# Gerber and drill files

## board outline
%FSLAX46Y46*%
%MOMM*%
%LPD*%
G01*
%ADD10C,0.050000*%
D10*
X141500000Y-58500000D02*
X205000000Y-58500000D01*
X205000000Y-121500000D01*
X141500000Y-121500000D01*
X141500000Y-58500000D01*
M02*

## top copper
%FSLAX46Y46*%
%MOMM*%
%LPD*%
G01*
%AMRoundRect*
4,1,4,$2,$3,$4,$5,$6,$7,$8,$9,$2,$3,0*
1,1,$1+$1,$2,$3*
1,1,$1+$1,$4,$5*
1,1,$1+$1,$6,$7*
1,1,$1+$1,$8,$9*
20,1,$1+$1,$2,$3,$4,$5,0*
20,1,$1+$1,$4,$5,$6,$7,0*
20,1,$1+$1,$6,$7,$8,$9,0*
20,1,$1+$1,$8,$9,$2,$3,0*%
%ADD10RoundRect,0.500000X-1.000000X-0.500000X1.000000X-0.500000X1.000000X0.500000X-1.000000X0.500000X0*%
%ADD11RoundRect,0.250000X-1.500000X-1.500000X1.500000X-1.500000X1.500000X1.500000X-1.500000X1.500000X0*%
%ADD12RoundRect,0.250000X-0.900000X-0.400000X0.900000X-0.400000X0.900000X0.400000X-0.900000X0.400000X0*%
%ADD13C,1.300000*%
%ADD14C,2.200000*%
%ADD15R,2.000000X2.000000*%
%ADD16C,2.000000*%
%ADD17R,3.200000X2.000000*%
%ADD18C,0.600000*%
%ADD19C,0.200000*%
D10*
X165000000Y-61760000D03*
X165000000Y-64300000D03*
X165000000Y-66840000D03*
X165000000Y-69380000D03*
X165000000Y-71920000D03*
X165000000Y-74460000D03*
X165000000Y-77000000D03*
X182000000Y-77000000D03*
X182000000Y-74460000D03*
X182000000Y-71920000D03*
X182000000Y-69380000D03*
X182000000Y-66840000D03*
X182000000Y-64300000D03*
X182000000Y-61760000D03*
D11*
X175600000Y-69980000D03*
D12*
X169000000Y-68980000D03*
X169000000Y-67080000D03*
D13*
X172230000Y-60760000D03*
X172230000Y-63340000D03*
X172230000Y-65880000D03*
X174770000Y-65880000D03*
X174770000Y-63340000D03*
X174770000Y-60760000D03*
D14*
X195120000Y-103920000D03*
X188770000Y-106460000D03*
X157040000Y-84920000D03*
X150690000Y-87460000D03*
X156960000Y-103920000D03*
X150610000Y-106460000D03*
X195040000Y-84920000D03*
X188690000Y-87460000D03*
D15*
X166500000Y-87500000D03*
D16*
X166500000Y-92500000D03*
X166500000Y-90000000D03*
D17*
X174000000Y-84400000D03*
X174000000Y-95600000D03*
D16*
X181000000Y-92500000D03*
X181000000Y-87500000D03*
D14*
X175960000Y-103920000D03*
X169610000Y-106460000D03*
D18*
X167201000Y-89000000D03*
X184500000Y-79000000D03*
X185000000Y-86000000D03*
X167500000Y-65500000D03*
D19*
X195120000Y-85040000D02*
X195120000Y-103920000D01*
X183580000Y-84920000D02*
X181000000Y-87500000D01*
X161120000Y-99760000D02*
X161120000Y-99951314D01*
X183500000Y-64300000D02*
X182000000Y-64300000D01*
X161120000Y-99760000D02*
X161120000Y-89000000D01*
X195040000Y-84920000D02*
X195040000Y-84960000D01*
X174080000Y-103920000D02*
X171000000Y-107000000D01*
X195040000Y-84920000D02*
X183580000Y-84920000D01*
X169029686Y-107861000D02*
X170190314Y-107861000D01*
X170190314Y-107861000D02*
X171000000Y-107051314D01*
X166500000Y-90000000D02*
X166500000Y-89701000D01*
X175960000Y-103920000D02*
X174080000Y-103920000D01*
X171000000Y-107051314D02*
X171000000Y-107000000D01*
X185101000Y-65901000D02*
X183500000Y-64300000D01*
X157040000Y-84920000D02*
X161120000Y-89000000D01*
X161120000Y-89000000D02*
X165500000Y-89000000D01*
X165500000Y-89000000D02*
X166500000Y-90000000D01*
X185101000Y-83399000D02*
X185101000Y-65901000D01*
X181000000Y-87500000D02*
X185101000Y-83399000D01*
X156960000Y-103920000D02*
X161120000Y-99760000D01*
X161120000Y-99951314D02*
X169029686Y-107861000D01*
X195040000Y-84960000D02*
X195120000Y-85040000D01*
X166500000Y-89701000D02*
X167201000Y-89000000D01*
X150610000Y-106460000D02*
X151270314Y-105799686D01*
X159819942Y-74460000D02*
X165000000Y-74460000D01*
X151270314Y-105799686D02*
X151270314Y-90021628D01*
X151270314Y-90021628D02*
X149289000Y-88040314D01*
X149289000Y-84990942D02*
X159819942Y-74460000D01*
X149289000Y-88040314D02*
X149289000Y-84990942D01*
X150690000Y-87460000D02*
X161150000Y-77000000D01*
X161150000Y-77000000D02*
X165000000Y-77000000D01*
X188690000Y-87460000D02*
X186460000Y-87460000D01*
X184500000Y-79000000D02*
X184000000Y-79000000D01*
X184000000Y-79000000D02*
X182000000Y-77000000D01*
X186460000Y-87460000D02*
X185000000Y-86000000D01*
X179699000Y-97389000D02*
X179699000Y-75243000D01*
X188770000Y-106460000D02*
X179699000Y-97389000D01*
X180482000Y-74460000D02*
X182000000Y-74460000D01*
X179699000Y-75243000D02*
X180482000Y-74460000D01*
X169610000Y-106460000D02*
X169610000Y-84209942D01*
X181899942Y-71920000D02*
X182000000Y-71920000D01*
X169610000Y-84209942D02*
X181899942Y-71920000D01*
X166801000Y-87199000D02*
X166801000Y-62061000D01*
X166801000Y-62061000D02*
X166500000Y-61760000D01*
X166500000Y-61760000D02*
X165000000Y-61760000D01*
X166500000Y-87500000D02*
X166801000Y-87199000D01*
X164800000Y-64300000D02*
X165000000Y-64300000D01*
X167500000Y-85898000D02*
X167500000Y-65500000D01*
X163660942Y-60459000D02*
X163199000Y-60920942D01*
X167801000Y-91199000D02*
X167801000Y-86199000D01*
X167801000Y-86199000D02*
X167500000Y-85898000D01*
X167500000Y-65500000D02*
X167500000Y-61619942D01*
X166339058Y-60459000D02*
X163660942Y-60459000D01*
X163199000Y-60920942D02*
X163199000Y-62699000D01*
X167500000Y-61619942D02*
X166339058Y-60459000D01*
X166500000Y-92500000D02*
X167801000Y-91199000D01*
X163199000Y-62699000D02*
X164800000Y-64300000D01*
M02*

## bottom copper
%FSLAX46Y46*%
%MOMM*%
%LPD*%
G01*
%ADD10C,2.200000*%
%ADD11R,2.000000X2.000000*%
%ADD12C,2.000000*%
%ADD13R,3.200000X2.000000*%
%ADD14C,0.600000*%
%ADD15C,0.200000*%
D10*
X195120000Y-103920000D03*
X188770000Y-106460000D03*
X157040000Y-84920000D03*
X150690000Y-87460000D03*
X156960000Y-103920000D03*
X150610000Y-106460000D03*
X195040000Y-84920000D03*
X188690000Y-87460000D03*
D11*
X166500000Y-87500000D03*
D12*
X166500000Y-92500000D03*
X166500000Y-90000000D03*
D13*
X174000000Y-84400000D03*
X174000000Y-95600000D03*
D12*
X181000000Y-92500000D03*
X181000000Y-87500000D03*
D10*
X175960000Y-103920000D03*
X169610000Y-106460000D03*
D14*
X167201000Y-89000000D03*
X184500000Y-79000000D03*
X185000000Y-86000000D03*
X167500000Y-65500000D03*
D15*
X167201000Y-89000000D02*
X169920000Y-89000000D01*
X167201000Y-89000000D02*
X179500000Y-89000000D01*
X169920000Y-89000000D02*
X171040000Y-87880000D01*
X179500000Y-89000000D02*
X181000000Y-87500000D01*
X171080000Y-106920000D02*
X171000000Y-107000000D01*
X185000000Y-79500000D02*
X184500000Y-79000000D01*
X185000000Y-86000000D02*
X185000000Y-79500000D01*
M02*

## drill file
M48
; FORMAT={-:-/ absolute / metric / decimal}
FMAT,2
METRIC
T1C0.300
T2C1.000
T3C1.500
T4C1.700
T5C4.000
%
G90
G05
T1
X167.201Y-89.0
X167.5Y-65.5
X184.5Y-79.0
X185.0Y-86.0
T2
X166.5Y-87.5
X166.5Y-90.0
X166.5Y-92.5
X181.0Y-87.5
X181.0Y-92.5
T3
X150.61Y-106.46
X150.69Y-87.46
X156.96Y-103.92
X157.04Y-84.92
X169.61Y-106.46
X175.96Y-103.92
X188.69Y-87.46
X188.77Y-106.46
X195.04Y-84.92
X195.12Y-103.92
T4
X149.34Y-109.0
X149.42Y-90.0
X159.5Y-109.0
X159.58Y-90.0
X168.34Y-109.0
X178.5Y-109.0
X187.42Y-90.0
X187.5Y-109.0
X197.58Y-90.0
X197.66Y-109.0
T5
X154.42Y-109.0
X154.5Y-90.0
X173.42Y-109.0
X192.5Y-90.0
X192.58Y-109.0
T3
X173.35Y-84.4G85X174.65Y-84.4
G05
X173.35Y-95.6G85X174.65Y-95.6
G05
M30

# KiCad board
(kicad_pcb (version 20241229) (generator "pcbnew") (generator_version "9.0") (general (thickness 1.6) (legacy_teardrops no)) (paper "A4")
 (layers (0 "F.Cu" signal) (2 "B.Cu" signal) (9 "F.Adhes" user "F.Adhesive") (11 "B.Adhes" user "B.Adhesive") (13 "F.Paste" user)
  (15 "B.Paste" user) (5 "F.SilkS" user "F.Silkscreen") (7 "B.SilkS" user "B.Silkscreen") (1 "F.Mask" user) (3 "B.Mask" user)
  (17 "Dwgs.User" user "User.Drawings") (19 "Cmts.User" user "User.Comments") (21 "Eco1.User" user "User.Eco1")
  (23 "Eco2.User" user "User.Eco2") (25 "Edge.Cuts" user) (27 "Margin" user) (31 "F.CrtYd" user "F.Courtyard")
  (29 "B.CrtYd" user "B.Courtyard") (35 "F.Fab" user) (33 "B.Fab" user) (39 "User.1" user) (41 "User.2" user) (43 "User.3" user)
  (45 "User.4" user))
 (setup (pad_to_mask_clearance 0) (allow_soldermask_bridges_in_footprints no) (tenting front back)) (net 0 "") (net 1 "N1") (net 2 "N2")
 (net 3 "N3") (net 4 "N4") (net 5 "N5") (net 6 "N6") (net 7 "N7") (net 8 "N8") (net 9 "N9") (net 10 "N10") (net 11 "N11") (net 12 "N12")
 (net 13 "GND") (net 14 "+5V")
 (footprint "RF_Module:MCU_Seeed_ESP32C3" (layer "F.Cu") (at 173.5 69.38)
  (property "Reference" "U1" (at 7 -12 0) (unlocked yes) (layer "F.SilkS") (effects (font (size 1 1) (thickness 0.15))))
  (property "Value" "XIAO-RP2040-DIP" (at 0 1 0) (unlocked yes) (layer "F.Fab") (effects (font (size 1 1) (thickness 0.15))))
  (pad "" smd roundrect (at 1.1 -0.4) (size 1.5 1.5) (layers "F.Paste") (roundrect_rratio 0.1666666667))
  (pad "" smd roundrect (at 1.1 1.6) (size 1.5 1.5) (layers "F.Paste") (roundrect_rratio 0.1666666667))
  (pad "" smd roundrect (at 3.1 -0.4) (size 1.5 1.5) (layers "F.Paste") (roundrect_rratio 0.1666666667))
  (pad "" smd roundrect (at 3.1 1.6) (size 1.5 1.5) (layers "F.Paste") (roundrect_rratio 0.1666666667))
  (pad "1" smd roundrect (at -8.5 -7.62) (size 3 2) (layers "F.Cu" "F.Mask" "F.Paste") (roundrect_rratio 0.25) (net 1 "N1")
   (thermal_bridge_angle 45))
  (pad "2" smd roundrect (at -8.5 -5.08) (size 3 2) (layers "F.Cu" "F.Mask" "F.Paste") (roundrect_rratio 0.25) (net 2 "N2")
   (thermal_bridge_angle 45))
  (pad "3" smd roundrect (at -8.5 -2.54) (size 3 2) (layers "F.Cu" "F.Mask" "F.Paste") (roundrect_rratio 0.25) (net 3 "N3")
   (thermal_bridge_angle 45))
  (pad "4" smd roundrect (at -8.5 0) (size 3 2) (layers "F.Cu" "F.Mask" "F.Paste") (roundrect_rratio 0.25) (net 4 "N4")
   (thermal_bridge_angle 45))
  (pad "5" smd roundrect (at -8.5 2.54) (size 3 2) (layers "F.Cu" "F.Mask" "F.Paste") (roundrect_rratio 0.25) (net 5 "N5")
   (thermal_bridge_angle 45))
  (pad "6" smd roundrect (at -8.5 5.08) (size 3 2) (layers "F.Cu" "F.Mask" "F.Paste") (roundrect_rratio 0.25) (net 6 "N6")
   (thermal_bridge_angle 45))
  (pad "7" smd roundrect (at -8.5 7.62) (size 3 2) (layers "F.Cu" "F.Mask" "F.Paste") (roundrect_rratio 0.25) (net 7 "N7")
   (thermal_bridge_angle 45))
  (pad "8" smd roundrect (at 8.5 7.62) (size 3 2) (layers "F.Cu" "F.Mask" "F.Paste") (roundrect_rratio 0.25) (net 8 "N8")
   (thermal_bridge_angle 45))
  (pad "9" smd roundrect (at 8.5 5.08) (size 3 2) (layers "F.Cu" "F.Mask" "F.Paste") (roundrect_rratio 0.25) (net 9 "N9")
   (thermal_bridge_angle 45))
  (pad "10" smd roundrect (at 8.5 2.54) (size 3 2) (layers "F.Cu" "F.Mask" "F.Paste") (roundrect_rratio 0.25) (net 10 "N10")
   (thermal_bridge_angle 45))
  (pad "11" smd roundrect (at 8.5 0) (size 3 2) (layers "F.Cu" "F.Mask" "F.Paste") (roundrect_rratio 0.25) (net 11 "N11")
   (thermal_bridge_angle 45))
  (pad "12" smd roundrect (at 8.5 -2.54) (size 3 2) (layers "F.Cu" "F.Mask" "F.Paste") (roundrect_rratio 0.25) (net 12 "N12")
   (thermal_bridge_angle 45))
  (pad "13" smd roundrect (at 8.5 -5.08) (size 3 2) (layers "F.Cu" "F.Mask" "F.Paste") (roundrect_rratio 0.25) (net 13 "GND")
   (thermal_bridge_angle 45))
  (pad "14" smd roundrect (at 8.5 -7.62) (size 3 2) (layers "F.Cu" "F.Mask" "F.Paste") (roundrect_rratio 0.25) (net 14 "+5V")
   (thermal_bridge_angle 45))
  (pad "15" smd roundrect (at 2.1 0.6) (size 3.5 3.5) (layers "F.Cu" "F.Mask") (roundrect_rratio 0.07142857143))
  (pad "16" smd roundrect (at -4.5 -0.4) (size 2.3 1.3) (layers "F.Cu" "F.Mask" "F.Paste") (roundrect_rratio 0.1923076923))
  (pad "17" smd roundrect (at -4.5 -2.3) (size 2.3 1.3) (layers "F.Cu" "F.Mask" "F.Paste") (roundrect_rratio 0.1923076923))
  (pad "18" smd circle (at -1.27 -8.62) (size 1.3 1.3) (layers "F.Cu" "F.Mask" "F.Paste"))
  (pad "19" smd circle (at -1.27 -6.04) (size 1.3 1.3) (layers "F.Cu" "F.Mask" "F.Paste"))
  (pad "20" smd circle (at -1.27 -3.5) (size 1.3 1.3) (layers "F.Cu" "F.Mask" "F.Paste"))
  (pad "21" smd circle (at 1.27 -3.5) (size 1.3 1.3) (layers "F.Cu" "F.Mask" "F.Paste"))
  (pad "22" smd circle (at 1.27 -6.04) (size 1.3 1.3) (layers "F.Cu" "F.Mask" "F.Paste"))
  (pad "23" smd circle (at 1.27 -8.62) (size 1.3 1.3) (layers "F.Cu" "F.Mask" "F.Paste")))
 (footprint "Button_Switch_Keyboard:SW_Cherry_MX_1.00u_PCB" (layer "F.Cu") (at 195.12 103.92)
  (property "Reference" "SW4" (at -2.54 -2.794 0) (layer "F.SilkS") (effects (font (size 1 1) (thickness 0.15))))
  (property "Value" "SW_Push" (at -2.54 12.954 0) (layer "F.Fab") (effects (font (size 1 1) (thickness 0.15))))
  (pad "" np_thru_hole circle (at -7.62 5.08) (size 1.7 1.7) (drill 1.7) (layers "*.Cu" "*.Mask"))
  (pad "" np_thru_hole circle (at -2.54 5.08) (size 4 4) (drill 4) (layers "*.Cu" "*.Mask"))
  (pad "" np_thru_hole circle (at 2.54 5.08) (size 1.7 1.7) (drill 1.7) (layers "*.Cu" "*.Mask"))
  (pad "1" thru_hole circle (at 0 0) (size 2.2 2.2) (drill 1.5) (layers "*.Cu" "*.Mask") (remove_unused_layers no) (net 13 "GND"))
  (pad "2" thru_hole circle (at -6.35 2.54) (size 2.2 2.2) (drill 1.5) (layers "*.Cu" "*.Mask") (remove_unused_layers no) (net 9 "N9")))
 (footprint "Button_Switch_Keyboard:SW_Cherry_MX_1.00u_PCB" (layer "F.Cu") (at 157.04 84.92)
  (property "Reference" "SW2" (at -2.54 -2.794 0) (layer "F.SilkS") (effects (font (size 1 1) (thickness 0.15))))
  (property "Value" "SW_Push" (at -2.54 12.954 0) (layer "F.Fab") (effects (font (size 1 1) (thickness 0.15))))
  (pad "" np_thru_hole circle (at -7.62 5.08) (size 1.7 1.7) (drill 1.7) (layers "*.Cu" "*.Mask"))
  (pad "" np_thru_hole circle (at -2.54 5.08) (size 4 4) (drill 4) (layers "*.Cu" "*.Mask"))
  (pad "" np_thru_hole circle (at 2.54 5.08) (size 1.7 1.7) (drill 1.7) (layers "*.Cu" "*.Mask"))
  (pad "1" thru_hole circle (at 0 0) (size 2.2 2.2) (drill 1.5) (layers "*.Cu" "*.Mask") (remove_unused_layers no) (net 13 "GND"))
  (pad "2" thru_hole circle (at -6.35 2.54) (size 2.2 2.2) (drill 1.5) (layers "*.Cu" "*.Mask") (remove_unused_layers no) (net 7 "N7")))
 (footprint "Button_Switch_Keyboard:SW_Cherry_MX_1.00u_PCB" (layer "F.Cu") (at 156.96 103.92)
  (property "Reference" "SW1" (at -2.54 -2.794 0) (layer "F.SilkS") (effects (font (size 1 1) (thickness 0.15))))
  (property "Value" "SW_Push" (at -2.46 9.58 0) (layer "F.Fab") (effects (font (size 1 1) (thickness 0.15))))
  (pad "" np_thru_hole circle (at -7.62 5.08) (size 1.7 1.7) (drill 1.7) (layers "*.Cu" "*.Mask"))
  (pad "" np_thru_hole circle (at -2.54 5.08) (size 4 4) (drill 4) (layers "*.Cu" "*.Mask"))
  (pad "" np_thru_hole circle (at 2.54 5.08) (size 1.7 1.7) (drill 1.7) (layers "*.Cu" "*.Mask"))
  (pad "1" thru_hole circle (at 0 0) (size 2.2 2.2) (drill 1.5) (layers "*.Cu" "*.Mask") (remove_unused_layers no) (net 13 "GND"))
  (pad "2" thru_hole circle (at -6.35 2.54) (size 2.2 2.2) (drill 1.5) (layers "*.Cu" "*.Mask") (remove_unused_layers no) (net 6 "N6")))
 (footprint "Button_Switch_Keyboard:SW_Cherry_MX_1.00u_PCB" (layer "F.Cu") (at 195.04 84.92)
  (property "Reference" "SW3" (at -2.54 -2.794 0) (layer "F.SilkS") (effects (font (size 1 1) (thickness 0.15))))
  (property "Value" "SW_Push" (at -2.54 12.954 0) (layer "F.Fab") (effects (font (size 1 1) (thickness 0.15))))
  (pad "" np_thru_hole circle (at -7.62 5.08) (size 1.7 1.7) (drill 1.7) (layers "*.Cu" "*.Mask"))
  (pad "" np_thru_hole circle (at -2.54 5.08) (size 4 4) (drill 4) (layers "*.Cu" "*.Mask"))
  (pad "" np_thru_hole circle (at 2.54 5.08) (size 1.7 1.7) (drill 1.7) (layers "*.Cu" "*.Mask"))
  (pad "1" thru_hole circle (at 0 0) (size 2.2 2.2) (drill 1.5) (layers "*.Cu" "*.Mask") (remove_unused_layers no) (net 13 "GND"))
  (pad "2" thru_hole circle (at -6.35 2.54) (size 2.2 2.2) (drill 1.5) (layers "*.Cu" "*.Mask") (remove_unused_layers no) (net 8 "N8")))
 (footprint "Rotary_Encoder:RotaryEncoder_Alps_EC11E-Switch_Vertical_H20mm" (layer "F.Cu") (at 166.5 87.5)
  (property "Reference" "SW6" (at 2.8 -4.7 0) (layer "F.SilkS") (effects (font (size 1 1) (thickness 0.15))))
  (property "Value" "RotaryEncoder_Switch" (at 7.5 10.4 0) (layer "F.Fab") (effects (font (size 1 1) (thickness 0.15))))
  (pad "A" thru_hole rect (at 0 0) (size 2 2) (drill 1) (layers "*.Cu" "*.Mask") (remove_unused_layers no) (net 1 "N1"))
  (pad "B" thru_hole circle (at 0 5) (size 2 2) (drill 1) (layers "*.Cu" "*.Mask") (remove_unused_layers no) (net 2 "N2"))
  (pad "C" thru_hole circle (at 0 2.5) (size 2 2) (drill 1) (layers "*.Cu" "*.Mask") (remove_unused_layers no) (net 13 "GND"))
  (pad "MP" thru_hole rect (at 7.5 -3.1) (size 3.2 2) (drill oval 2.8 1.5) (layers "*.Cu" "*.Mask") (remove_unused_layers no))
  (pad "MP" thru_hole rect (at 7.5 8.1) (size 3.2 2) (drill oval 2.8 1.5) (layers "*.Cu" "*.Mask") (remove_unused_layers no))
  (pad "S1" thru_hole circle (at 14.5 5) (size 2 2) (drill 1) (layers "*.Cu" "*.Mask") (remove_unused_layers no) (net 11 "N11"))
  (pad "S2" thru_hole circle (at 14.5 0) (size 2 2) (drill 1) (layers "*.Cu" "*.Mask") (remove_unused_layers no) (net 13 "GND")))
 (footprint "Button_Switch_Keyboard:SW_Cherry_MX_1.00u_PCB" (layer "F.Cu") (at 175.96 103.92)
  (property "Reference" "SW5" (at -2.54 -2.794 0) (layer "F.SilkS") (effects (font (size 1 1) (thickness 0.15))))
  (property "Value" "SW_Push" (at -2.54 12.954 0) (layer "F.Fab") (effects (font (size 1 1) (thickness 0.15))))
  (pad "" np_thru_hole circle (at -7.62 5.08) (size 1.7 1.7) (drill 1.7) (layers "*.Cu" "*.Mask"))
  (pad "" np_thru_hole circle (at -2.54 5.08) (size 4 4) (drill 4) (layers "*.Cu" "*.Mask"))
  (pad "" np_thru_hole circle (at 2.54 5.08) (size 1.7 1.7) (drill 1.7) (layers "*.Cu" "*.Mask"))
  (pad "1" thru_hole circle (at 0 0) (size 2.2 2.2) (drill 1.5) (layers "*.Cu" "*.Mask") (remove_unused_layers no) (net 13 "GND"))
  (pad "2" thru_hole circle (at -6.35 2.54) (size 2.2 2.2) (drill 1.5) (layers "*.Cu" "*.Mask") (remove_unused_layers no) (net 10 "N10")))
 (gr_rect (start 141.5 58.5) (end 205 121.5) (stroke (width 0.05) (type default)) (fill no) (layer "Edge.Cuts"))
 (segment (start 195.12 85.04) (end 195.12 103.92) (width 0.2) (layer "F.Cu") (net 13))
 (segment (start 183.58 84.92) (end 181 87.5) (width 0.2) (layer "F.Cu") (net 13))
 (segment (start 161.12 99.76) (end 161.12 99.951314) (width 0.2) (layer "F.Cu") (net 13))
 (segment (start 183.5 64.3) (end 182 64.3) (width 0.2) (layer "F.Cu") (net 13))
 (segment (start 161.12 99.76) (end 161.12 89) (width 0.2) (layer "F.Cu") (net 13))
 (segment (start 195.04 84.92) (end 195.04 84.96) (width 0.2) (layer "F.Cu") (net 13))
 (segment (start 174.08 103.92) (end 171 107) (width 0.2) (layer "F.Cu") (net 13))
 (segment (start 195.04 84.92) (end 183.58 84.92) (width 0.2) (layer "F.Cu") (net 13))
 (segment (start 169.029686 107.861) (end 170.190314 107.861) (width 0.2) (layer "F.Cu") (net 13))
 (segment (start 170.190314 107.861) (end 171 107.051314) (width 0.2) (layer "F.Cu") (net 13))
 (segment (start 166.5 90) (end 166.5 89.701) (width 0.2) (layer "F.Cu") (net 13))
 (segment (start 175.96 103.92) (end 174.08 103.92) (width 0.2) (layer "F.Cu") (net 13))
 (segment (start 171 107.051314) (end 171 107) (width 0.2) (layer "F.Cu") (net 13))
 (segment (start 185.101 65.901) (end 183.5 64.3) (width 0.2) (layer "F.Cu") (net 13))
 (segment (start 157.04 84.92) (end 161.12 89) (width 0.2) (layer "F.Cu") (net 13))
 (segment (start 161.12 89) (end 165.5 89) (width 0.2) (layer "F.Cu") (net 13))
 (segment (start 165.5 89) (end 166.5 90) (width 0.2) (layer "F.Cu") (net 13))
 (segment (start 185.101 83.399) (end 185.101 65.901) (width 0.2) (layer "F.Cu") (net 13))
 (segment (start 181 87.5) (end 185.101 83.399) (width 0.2) (layer "F.Cu") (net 13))
 (segment (start 156.96 103.92) (end 161.12 99.76) (width 0.2) (layer "F.Cu") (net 13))
 (segment (start 161.12 99.951314) (end 169.029686 107.861) (width 0.2) (layer "F.Cu") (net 13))
 (segment (start 195.04 84.96) (end 195.12 85.04) (width 0.2) (layer "F.Cu") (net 13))
 (segment (start 166.5 89.701) (end 167.201 89) (width 0.2) (layer "F.Cu") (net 13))
 (via (at 167.201 89) (size 0.6) (drill 0.3) (layers "F.Cu" "B.Cu") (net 13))
 (segment (start 167.201 89) (end 169.92 89) (width 0.2) (layer "B.Cu") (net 13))
 (segment (start 167.201 89) (end 179.5 89) (width 0.2) (layer "B.Cu") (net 13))
 (segment (start 169.92 89) (end 171.04 87.88) (width 0.2) (layer "B.Cu") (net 13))
 (segment (start 179.5 89) (end 181 87.5) (width 0.2) (layer "B.Cu") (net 13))
 (segment (start 171.08 106.92) (end 171 107) (width 0.2) (layer "B.Cu") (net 13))
 (segment (start 150.61 106.46) (end 151.270314 105.799686) (width 0.2) (layer "F.Cu") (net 6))
 (segment (start 159.819942 74.46) (end 165 74.46) (width 0.2) (layer "F.Cu") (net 6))
 (segment (start 151.270314 105.799686) (end 151.270314 90.021628) (width 0.2) (layer "F.Cu") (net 6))
 (segment (start 151.270314 90.021628) (end 149.289 88.040314) (width 0.2) (layer "F.Cu") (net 6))
 (segment (start 149.289 84.990942) (end 159.819942 74.46) (width 0.2) (layer "F.Cu") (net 6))
 (segment (start 149.289 88.040314) (end 149.289 84.990942) (width 0.2) (layer "F.Cu") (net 6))
 (segment (start 150.69 87.46) (end 161.15 77) (width 0.2) (layer "F.Cu") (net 7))
 (segment (start 161.15 77) (end 165 77) (width 0.2) (layer "F.Cu") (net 7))
 (segment (start 188.69 87.46) (end 186.46 87.46) (width 0.2) (layer "F.Cu") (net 8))
 (segment (start 184.5 79) (end 184 79) (width 0.2) (layer "F.Cu") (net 8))
 (segment (start 184 79) (end 182 77) (width 0.2) (layer "F.Cu") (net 8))
 (segment (start 186.46 87.46) (end 185 86) (width 0.2) (layer "F.Cu") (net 8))
 (via (at 184.5 79) (size 0.6) (drill 0.3) (layers "F.Cu" "B.Cu") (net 8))
 (via (at 185 86) (size 0.6) (drill 0.3) (layers "F.Cu" "B.Cu") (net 8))
 (segment (start 185 79.5) (end 184.5 79) (width 0.2) (layer "B.Cu") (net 8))
 (segment (start 185 86) (end 185 79.5) (width 0.2) (layer "B.Cu") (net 8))
 (segment (start 179.699 97.389) (end 179.699 75.243) (width 0.2) (layer "F.Cu") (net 9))
 (segment (start 188.77 106.46) (end 179.699 97.389) (width 0.2) (layer "F.Cu") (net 9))
 (segment (start 180.482 74.46) (end 182 74.46) (width 0.2) (layer "F.Cu") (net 9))
 (segment (start 179.699 75.243) (end 180.482 74.46) (width 0.2) (layer "F.Cu") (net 9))
 (segment (start 169.61 106.46) (end 169.61 84.209942) (width 0.2) (layer "F.Cu") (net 10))
 (segment (start 181.899942 71.92) (end 182 71.92) (width 0.2) (layer "F.Cu") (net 10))
 (segment (start 169.61 84.209942) (end 181.899942 71.92) (width 0.2) (layer "F.Cu") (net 10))
 (segment (start 166.801 87.199) (end 166.801 62.061) (width 0.2) (layer "F.Cu") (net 1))
 (segment (start 166.801 62.061) (end 166.5 61.76) (width 0.2) (layer "F.Cu") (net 1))
 (segment (start 166.5 61.76) (end 165 61.76) (width 0.2) (layer "F.Cu") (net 1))
 (segment (start 166.5 87.5) (end 166.801 87.199) (width 0.2) (layer "F.Cu") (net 1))
 (segment (start 164.8 64.3) (end 165 64.3) (width 0.2) (layer "F.Cu") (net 2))
 (segment (start 167.5 85.898) (end 167.5 65.5) (width 0.2) (layer "F.Cu") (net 2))
 (segment (start 163.660942 60.459) (end 163.199 60.920942) (width 0.2) (layer "F.Cu") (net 2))
 (segment (start 167.801 91.199) (end 167.801 86.199) (width 0.2) (layer "F.Cu") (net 2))
 (segment (start 167.801 86.199) (end 167.5 85.898) (width 0.2) (layer "F.Cu") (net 2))
 (segment (start 167.5 65.5) (end 167.5 61.619942) (width 0.2) (layer "F.Cu") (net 2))
 (segment (start 166.339058 60.459) (end 163.660942 60.459) (width 0.2) (layer "F.Cu") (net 2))
 (segment (start 163.199 60.920942) (end 163.199 62.699) (width 0.2) (layer "F.Cu") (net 2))
 (segment (start 167.5 61.619942) (end 166.339058 60.459) (width 0.2) (layer "F.Cu") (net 2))
 (segment (start 166.5 92.5) (end 167.801 91.199) (width 0.2) (layer "F.Cu") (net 2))
 (segment (start 163.199 62.699) (end 164.8 64.3) (width 0.2) (layer "F.Cu") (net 2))
 (via (at 167.5 65.5) (size 0.6) (drill 0.3) (layers "F.Cu" "B.Cu") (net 2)))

